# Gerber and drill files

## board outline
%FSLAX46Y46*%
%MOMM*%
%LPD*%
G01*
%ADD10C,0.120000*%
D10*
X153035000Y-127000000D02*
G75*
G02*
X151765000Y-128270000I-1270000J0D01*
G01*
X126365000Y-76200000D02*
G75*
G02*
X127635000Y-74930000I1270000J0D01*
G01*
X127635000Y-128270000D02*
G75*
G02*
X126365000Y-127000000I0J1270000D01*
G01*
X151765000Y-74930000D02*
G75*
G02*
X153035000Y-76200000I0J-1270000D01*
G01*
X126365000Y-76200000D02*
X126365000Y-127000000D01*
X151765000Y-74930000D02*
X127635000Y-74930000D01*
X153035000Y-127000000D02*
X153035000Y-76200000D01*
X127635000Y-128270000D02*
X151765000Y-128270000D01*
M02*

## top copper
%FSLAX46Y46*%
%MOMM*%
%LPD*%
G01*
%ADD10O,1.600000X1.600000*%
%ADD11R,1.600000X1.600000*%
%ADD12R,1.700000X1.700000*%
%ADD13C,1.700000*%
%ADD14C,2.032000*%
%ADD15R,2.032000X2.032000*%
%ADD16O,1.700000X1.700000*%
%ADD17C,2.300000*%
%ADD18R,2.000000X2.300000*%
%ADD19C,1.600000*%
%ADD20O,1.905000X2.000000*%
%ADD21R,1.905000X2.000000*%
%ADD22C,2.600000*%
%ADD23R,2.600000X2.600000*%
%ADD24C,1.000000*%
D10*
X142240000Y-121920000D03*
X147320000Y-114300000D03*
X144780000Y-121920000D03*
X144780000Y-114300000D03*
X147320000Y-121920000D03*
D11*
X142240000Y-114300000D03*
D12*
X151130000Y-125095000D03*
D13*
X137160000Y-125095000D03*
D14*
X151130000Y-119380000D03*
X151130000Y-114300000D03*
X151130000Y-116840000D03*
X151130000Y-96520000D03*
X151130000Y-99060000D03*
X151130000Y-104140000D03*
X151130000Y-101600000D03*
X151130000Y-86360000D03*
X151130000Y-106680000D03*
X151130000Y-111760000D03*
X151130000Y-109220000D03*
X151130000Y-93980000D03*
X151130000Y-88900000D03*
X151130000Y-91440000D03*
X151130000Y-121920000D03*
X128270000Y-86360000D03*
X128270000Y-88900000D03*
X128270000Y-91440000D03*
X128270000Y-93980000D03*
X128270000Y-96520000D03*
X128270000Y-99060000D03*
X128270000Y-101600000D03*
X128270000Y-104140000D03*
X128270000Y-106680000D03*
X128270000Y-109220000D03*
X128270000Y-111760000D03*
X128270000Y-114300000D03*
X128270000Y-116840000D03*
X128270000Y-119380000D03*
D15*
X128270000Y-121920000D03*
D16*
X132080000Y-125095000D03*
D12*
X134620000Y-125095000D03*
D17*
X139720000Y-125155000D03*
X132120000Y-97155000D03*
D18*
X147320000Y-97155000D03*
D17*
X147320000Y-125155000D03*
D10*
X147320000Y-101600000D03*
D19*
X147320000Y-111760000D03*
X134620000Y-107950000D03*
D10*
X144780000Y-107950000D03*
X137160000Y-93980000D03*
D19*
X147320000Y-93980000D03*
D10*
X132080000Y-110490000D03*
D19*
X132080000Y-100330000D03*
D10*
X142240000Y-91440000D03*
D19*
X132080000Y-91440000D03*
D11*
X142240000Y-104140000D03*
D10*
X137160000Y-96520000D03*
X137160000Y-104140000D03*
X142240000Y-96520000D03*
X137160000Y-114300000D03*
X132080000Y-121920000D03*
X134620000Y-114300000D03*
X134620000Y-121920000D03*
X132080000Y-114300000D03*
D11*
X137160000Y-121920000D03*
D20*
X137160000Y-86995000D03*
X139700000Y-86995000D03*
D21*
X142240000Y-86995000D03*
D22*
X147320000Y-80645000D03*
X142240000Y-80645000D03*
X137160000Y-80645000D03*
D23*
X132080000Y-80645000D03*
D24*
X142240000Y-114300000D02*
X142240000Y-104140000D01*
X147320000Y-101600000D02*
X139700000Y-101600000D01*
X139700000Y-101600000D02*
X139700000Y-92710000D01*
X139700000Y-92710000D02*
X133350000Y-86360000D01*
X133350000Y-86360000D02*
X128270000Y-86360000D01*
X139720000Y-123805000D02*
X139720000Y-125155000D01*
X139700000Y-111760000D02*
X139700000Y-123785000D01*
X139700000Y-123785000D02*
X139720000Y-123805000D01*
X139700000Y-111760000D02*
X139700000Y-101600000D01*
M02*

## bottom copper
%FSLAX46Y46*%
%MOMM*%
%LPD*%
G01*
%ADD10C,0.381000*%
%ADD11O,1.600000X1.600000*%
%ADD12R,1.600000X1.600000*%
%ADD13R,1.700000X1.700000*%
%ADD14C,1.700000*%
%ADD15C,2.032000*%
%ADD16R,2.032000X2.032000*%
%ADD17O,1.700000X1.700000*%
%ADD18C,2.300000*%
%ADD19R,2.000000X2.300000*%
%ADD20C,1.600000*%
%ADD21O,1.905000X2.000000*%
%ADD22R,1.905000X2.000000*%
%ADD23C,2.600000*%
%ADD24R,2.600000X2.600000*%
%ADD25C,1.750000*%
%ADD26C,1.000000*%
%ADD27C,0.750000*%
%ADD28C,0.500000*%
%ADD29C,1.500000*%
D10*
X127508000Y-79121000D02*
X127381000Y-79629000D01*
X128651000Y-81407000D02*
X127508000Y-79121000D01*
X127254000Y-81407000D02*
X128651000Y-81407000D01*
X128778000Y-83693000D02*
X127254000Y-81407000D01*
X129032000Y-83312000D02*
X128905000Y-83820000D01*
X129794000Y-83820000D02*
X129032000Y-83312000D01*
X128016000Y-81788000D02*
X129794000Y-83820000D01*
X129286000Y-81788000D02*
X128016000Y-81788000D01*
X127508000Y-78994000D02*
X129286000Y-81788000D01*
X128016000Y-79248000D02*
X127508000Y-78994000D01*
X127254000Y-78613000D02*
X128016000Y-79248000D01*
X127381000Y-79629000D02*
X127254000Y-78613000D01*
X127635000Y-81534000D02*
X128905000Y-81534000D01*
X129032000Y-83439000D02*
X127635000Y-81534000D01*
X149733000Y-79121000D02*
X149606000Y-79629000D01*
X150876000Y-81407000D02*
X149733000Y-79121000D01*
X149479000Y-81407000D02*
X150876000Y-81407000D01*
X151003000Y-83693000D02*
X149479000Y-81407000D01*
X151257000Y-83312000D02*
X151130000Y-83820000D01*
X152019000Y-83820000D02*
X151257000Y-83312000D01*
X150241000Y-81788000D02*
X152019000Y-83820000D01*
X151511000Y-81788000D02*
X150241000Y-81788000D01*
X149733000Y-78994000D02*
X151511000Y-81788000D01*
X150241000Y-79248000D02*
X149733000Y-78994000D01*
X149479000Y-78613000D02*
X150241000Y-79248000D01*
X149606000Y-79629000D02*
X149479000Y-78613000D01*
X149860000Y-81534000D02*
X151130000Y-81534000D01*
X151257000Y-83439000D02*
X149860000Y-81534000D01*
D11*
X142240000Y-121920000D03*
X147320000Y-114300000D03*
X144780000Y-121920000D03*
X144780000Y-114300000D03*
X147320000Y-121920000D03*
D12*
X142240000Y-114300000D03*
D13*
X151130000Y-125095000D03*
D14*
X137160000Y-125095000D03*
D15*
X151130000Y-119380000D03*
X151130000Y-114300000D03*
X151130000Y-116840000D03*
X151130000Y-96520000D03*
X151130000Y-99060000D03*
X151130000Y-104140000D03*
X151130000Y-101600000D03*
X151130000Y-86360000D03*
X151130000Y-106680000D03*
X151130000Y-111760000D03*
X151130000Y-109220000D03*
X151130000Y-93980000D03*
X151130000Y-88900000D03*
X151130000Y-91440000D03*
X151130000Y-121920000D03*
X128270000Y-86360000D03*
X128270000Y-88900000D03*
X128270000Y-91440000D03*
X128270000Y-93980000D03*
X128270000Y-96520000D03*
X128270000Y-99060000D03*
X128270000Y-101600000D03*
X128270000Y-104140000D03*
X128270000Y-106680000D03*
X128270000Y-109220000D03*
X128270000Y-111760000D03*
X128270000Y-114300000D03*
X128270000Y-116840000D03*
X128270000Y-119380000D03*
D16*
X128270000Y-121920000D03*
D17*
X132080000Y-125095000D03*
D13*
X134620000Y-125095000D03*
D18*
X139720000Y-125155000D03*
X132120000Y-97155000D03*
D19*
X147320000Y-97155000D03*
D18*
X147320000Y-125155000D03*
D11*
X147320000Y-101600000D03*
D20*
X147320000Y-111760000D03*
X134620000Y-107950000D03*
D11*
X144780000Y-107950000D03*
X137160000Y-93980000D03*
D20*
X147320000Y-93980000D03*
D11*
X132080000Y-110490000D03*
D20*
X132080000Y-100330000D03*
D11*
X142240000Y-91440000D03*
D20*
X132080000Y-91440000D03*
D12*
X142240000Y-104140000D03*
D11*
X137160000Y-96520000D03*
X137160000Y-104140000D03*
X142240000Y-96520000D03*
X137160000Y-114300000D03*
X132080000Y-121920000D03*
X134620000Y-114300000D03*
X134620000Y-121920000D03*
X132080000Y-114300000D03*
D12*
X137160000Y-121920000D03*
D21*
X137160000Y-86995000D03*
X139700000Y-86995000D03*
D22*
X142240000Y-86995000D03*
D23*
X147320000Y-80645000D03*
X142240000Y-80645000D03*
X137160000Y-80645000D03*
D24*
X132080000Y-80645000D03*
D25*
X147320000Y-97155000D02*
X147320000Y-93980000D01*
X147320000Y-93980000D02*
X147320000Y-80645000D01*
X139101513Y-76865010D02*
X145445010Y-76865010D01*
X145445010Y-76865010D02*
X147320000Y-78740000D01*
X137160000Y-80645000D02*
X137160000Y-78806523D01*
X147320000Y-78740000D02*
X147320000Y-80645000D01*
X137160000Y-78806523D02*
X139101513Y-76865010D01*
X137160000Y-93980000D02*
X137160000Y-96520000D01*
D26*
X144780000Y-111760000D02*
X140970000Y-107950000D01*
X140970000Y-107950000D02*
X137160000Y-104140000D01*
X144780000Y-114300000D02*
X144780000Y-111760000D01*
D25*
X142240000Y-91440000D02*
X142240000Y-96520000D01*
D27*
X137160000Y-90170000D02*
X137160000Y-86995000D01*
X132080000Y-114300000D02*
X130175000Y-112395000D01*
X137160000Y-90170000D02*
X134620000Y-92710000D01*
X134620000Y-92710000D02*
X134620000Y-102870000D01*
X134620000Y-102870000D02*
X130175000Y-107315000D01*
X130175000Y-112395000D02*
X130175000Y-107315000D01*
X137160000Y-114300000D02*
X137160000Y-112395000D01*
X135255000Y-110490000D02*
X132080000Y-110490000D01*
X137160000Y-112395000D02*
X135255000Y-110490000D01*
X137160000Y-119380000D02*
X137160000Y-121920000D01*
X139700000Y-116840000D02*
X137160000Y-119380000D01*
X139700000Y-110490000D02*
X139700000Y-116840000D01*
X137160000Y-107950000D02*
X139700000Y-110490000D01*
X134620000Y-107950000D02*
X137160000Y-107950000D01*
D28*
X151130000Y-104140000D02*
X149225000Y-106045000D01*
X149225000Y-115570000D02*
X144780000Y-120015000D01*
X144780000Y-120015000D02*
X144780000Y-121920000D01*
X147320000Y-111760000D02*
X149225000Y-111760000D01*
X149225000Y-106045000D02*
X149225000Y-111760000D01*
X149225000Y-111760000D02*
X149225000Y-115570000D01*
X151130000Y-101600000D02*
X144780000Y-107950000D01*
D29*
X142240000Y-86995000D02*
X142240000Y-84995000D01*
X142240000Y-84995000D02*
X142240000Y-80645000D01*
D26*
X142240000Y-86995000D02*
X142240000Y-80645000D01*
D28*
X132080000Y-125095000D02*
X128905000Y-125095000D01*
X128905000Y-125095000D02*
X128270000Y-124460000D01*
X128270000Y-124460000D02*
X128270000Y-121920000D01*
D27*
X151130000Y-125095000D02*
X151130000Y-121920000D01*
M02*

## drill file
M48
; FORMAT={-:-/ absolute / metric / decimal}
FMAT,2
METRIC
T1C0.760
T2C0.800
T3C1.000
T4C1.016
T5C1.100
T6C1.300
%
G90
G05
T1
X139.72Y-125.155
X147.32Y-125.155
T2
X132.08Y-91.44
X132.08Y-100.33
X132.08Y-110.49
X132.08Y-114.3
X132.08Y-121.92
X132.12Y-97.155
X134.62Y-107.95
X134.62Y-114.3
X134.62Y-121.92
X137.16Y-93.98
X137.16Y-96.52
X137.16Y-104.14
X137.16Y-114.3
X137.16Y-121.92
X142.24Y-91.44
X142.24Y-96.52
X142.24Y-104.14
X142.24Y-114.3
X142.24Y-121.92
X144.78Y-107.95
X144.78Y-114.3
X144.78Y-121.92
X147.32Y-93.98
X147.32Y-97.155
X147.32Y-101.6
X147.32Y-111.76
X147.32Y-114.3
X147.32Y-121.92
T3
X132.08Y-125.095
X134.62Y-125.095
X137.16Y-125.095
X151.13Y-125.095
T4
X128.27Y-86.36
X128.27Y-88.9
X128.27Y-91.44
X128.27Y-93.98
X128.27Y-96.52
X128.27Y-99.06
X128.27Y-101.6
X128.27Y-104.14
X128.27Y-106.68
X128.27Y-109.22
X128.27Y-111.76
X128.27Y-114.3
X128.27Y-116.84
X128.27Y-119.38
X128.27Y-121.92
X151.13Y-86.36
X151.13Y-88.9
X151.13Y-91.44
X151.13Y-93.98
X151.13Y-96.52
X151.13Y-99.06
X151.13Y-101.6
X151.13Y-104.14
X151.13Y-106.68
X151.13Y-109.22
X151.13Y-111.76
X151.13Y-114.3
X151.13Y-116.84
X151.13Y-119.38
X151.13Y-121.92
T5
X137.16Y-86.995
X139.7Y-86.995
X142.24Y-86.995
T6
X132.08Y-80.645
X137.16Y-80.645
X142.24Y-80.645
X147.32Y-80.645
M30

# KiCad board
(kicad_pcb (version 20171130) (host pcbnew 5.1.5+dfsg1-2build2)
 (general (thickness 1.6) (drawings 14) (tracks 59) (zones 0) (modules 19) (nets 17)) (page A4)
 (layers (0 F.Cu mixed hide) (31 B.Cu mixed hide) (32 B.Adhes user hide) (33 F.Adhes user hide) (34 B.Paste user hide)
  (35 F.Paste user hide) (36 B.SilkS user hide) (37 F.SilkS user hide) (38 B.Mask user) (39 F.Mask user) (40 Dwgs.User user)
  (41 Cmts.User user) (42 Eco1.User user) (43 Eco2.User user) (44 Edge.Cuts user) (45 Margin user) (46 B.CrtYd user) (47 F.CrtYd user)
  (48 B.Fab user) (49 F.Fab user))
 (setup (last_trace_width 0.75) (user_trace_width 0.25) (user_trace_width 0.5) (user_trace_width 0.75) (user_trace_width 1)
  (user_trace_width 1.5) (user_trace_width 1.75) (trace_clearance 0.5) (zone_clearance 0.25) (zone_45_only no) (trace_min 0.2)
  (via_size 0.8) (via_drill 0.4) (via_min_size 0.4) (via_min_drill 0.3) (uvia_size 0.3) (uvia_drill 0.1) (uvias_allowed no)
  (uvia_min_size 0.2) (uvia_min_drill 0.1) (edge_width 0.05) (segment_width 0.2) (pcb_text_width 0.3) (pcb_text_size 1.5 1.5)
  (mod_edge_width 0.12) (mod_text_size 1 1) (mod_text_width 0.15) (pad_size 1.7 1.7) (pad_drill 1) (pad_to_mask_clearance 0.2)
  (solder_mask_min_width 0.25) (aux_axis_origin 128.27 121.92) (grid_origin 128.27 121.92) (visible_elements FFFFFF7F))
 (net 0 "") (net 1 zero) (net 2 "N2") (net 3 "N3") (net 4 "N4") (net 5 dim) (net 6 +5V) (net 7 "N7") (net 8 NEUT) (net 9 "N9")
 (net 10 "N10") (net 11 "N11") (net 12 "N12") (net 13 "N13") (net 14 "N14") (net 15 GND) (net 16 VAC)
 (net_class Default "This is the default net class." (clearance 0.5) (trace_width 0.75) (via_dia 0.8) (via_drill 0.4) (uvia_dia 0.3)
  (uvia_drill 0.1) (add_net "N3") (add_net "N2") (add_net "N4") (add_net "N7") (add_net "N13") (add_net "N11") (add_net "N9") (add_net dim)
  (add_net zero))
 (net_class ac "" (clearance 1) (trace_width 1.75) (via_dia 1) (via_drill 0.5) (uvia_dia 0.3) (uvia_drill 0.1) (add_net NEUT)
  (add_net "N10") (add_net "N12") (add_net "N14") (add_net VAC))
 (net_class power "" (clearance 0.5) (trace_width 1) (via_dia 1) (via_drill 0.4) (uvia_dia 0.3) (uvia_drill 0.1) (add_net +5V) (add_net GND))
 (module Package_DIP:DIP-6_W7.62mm (layer B.Cu) (at 142.24 114.3 270)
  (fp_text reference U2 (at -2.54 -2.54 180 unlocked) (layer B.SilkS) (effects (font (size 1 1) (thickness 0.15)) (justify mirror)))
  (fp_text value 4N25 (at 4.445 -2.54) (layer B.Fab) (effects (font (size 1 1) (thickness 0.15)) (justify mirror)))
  (pad 6 thru_hole oval (at 7.62 0 270) (size 1.6 1.6) (drill 0.8) (layers *.Cu *.Mask))
  (pad 3 thru_hole oval (at 0 -5.08 270) (size 1.6 1.6) (drill 0.8) (layers *.Cu *.Mask))
  (pad 5 thru_hole oval (at 7.62 -2.54 270) (size 1.6 1.6) (drill 0.8) (layers *.Cu *.Mask) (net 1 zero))
  (pad 2 thru_hole oval (at 0 -2.54 270) (size 1.6 1.6) (drill 0.8) (layers *.Cu *.Mask) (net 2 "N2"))
  (pad 4 thru_hole oval (at 7.62 -5.08 270) (size 1.6 1.6) (drill 0.8) (layers *.Cu *.Mask))
  (pad 1 thru_hole rect (at 0 0 270) (size 1.6 1.6) (drill 0.8) (layers *.Cu *.Mask) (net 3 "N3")))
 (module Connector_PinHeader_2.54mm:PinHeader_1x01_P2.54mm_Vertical (layer B.Cu) (at 151.13 125.095)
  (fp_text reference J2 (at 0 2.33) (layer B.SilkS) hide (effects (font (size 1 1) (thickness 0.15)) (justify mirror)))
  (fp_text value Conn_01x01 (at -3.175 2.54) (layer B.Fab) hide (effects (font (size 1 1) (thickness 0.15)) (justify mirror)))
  (pad 1 thru_hole rect (at 0 0) (size 1.7 1.7) (drill 1) (layers *.Cu *.Mask) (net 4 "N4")))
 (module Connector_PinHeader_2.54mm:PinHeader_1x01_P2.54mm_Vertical (layer B.Cu) (at 137.16 125.095)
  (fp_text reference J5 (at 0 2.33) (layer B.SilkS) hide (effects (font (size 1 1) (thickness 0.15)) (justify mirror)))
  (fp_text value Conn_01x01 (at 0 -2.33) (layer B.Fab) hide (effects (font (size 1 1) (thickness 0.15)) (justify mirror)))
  (pad 1 thru_hole circle (at 0 0) (size 1.7 1.7) (drill 1) (layers *.Cu *.Mask)))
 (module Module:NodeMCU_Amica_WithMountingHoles (layer B.Cu) (at 128.27 121.92)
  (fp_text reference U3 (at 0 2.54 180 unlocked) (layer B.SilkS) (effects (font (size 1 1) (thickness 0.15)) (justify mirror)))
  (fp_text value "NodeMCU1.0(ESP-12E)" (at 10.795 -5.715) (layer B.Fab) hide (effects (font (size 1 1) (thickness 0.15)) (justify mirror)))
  (pad 29 thru_hole circle (at 22.86 -2.54) (size 2.032 2.032) (drill 1.016) (layers *.Cu *.Mask))
  (pad 27 thru_hole circle (at 22.86 -7.62) (size 2.032 2.032) (drill 1.016) (layers *.Cu *.Mask))
  (pad 28 thru_hole circle (at 22.86 -5.08) (size 2.032 2.032) (drill 1.016) (layers *.Cu *.Mask))
  (pad 20 thru_hole circle (at 22.86 -25.4) (size 2.032 2.032) (drill 1.016) (layers *.Cu *.Mask))
  (pad 21 thru_hole circle (at 22.86 -22.86) (size 2.032 2.032) (drill 1.016) (layers *.Cu *.Mask))
  (pad 23 thru_hole circle (at 22.86 -17.78) (size 2.032 2.032) (drill 1.016) (layers *.Cu *.Mask) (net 1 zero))
  (pad 22 thru_hole circle (at 22.86 -20.32) (size 2.032 2.032) (drill 1.016) (layers *.Cu *.Mask) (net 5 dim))
  (pad 16 thru_hole circle (at 22.86 -35.56) (size 2.032 2.032) (drill 1.016) (layers *.Cu *.Mask))
  (pad 24 thru_hole circle (at 22.86 -15.24) (size 2.032 2.032) (drill 1.016) (layers *.Cu *.Mask))
  (pad 26 thru_hole circle (at 22.86 -10.16) (size 2.032 2.032) (drill 1.016) (layers *.Cu *.Mask))
  (pad 25 thru_hole circle (at 22.86 -12.7) (size 2.032 2.032) (drill 1.016) (layers *.Cu *.Mask))
  (pad 19 thru_hole circle (at 22.86 -27.94) (size 2.032 2.032) (drill 1.016) (layers *.Cu *.Mask))
  (pad 17 thru_hole circle (at 22.86 -33.02) (size 2.032 2.032) (drill 1.016) (layers *.Cu *.Mask))
  (pad 18 thru_hole circle (at 22.86 -30.48) (size 2.032 2.032) (drill 1.016) (layers *.Cu *.Mask))
  (pad 30 thru_hole circle (at 22.86 0) (size 2.032 2.032) (drill 1.016) (layers *.Cu *.Mask) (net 4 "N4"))
  (pad 15 thru_hole circle (at 0 -35.56) (size 2.032 2.032) (drill 1.016) (layers *.Cu *.Mask) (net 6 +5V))
  (pad 14 thru_hole circle (at 0 -33.02) (size 2.032 2.032) (drill 1.016) (layers *.Cu *.Mask))
  (pad 13 thru_hole circle (at 0 -30.48) (size 2.032 2.032) (drill 1.016) (layers *.Cu *.Mask))
  (pad 12 thru_hole circle (at 0 -27.94) (size 2.032 2.032) (drill 1.016) (layers *.Cu *.Mask))
  (pad 11 thru_hole circle (at 0 -25.4) (size 2.032 2.032) (drill 1.016) (layers *.Cu *.Mask))
  (pad 10 thru_hole circle (at 0 -22.86) (size 2.032 2.032) (drill 1.016) (layers *.Cu *.Mask))
  (pad 9 thru_hole circle (at 0 -20.32) (size 2.032 2.032) (drill 1.016) (layers *.Cu *.Mask))
  (pad 8 thru_hole circle (at 0 -17.78) (size 2.032 2.032) (drill 1.016) (layers *.Cu *.Mask))
  (pad 7 thru_hole circle (at 0 -15.24) (size 2.032 2.032) (drill 1.016) (layers *.Cu *.Mask))
  (pad 6 thru_hole circle (at 0 -12.7) (size 2.032 2.032) (drill 1.016) (layers *.Cu *.Mask))
  (pad 5 thru_hole circle (at 0 -10.16) (size 2.032 2.032) (drill 1.016) (layers *.Cu *.Mask))
  (pad 4 thru_hole circle (at 0 -7.62) (size 2.032 2.032) (drill 1.016) (layers *.Cu *.Mask))
  (pad 3 thru_hole circle (at 0 -5.08) (size 2.032 2.032) (drill 1.016) (layers *.Cu *.Mask))
  (pad 2 thru_hole circle (at 0 -2.54) (size 2.032 2.032) (drill 1.016) (layers *.Cu *.Mask))
  (pad 1 thru_hole rect (at 0 0) (size 2.032 2.032) (drill 1.016) (layers *.Cu *.Mask) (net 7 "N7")))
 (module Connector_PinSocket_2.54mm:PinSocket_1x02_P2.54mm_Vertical (layer B.Cu) (at 134.62 125.095 90)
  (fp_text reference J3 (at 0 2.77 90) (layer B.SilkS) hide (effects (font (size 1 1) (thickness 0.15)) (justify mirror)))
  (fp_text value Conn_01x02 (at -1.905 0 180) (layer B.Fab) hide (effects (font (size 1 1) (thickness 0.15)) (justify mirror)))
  (pad 2 thru_hole oval (at 0 -2.54 90) (size 1.7 1.7) (drill 1) (layers *.Cu *.Mask) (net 7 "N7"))
  (pad 1 thru_hole rect (at 0 0 90) (size 1.7 1.7) (drill 1) (layers *.Cu *.Mask)))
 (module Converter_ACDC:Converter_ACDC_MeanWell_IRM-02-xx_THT (layer F.Cu) (at 147.32 97.155 270)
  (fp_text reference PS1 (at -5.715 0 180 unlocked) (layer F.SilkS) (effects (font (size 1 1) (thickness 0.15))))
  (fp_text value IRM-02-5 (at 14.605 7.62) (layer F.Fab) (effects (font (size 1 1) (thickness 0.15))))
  (pad 4 thru_hole circle (at 28 7.6 270) (size 2.3 2.3) (drill 0.76) (layers *.Cu *.Mask) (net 6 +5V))
  (pad 2 thru_hole circle (at 0 15.2 270) (size 2.3 2.3) (drill 0.8) (layers *.Cu *.Mask))
  (pad 1 thru_hole rect (at 0 0 270) (size 2.3 2) (drill 0.8) (layers *.Cu *.Mask) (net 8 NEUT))
  (pad 3 thru_hole circle (at 28 0 270) (size 2.3 2.3) (drill 0.76) (layers *.Cu *.Mask)))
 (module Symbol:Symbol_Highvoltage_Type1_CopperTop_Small (layer B.Cu) (at 127.635 80.645)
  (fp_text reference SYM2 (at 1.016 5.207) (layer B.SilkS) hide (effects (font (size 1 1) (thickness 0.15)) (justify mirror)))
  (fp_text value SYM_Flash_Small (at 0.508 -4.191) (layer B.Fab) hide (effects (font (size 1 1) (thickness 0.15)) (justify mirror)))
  (fp_line (start -0.127 -1.524) (end -0.254 -1.016) (layer B.Cu) (width 0.381))
  (fp_line (start 1.016 0.762) (end -0.127 -1.524) (layer B.Cu) (width 0.381))
  (fp_line (start -0.381 0.762) (end 1.016 0.762) (layer B.Cu) (width 0.381))
  (fp_line (start 1.143 3.048) (end -0.381 0.762) (layer B.Cu) (width 0.381))
  (fp_line (start 1.397 2.667) (end 1.27 3.175) (layer B.Cu) (width 0.381))
  (fp_line (start 2.159 3.175) (end 1.397 2.667) (layer B.Cu) (width 0.381))
  (fp_line (start 0.381 1.143) (end 2.159 3.175) (layer B.Cu) (width 0.381))
  (fp_line (start 1.651 1.143) (end 0.381 1.143) (layer B.Cu) (width 0.381))
  (fp_line (start -0.127 -1.651) (end 1.651 1.143) (layer B.Cu) (width 0.381))
  (fp_line (start 0.381 -1.397) (end -0.127 -1.651) (layer B.Cu) (width 0.381))
  (fp_line (start -0.381 -2.032) (end 0.381 -1.397) (layer B.Cu) (width 0.381))
  (fp_line (start -0.254 -1.016) (end -0.381 -2.032) (layer B.Cu) (width 0.381))
  (fp_line (start 0 0.889) (end 1.27 0.889) (layer B.Cu) (width 0.381))
  (fp_line (start 1.397 2.794) (end 0 0.889) (layer B.Cu) (width 0.381)))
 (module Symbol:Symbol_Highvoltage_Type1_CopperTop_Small (layer B.Cu) (at 149.86 80.645)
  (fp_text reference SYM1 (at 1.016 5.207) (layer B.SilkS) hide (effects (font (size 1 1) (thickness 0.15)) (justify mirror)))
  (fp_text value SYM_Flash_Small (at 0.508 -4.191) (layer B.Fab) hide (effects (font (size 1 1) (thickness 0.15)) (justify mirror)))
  (fp_line (start -0.127 -1.524) (end -0.254 -1.016) (layer B.Cu) (width 0.381))
  (fp_line (start 1.016 0.762) (end -0.127 -1.524) (layer B.Cu) (width 0.381))
  (fp_line (start -0.381 0.762) (end 1.016 0.762) (layer B.Cu) (width 0.381))
  (fp_line (start 1.143 3.048) (end -0.381 0.762) (layer B.Cu) (width 0.381))
  (fp_line (start 1.397 2.667) (end 1.27 3.175) (layer B.Cu) (width 0.381))
  (fp_line (start 2.159 3.175) (end 1.397 2.667) (layer B.Cu) (width 0.381))
  (fp_line (start 0.381 1.143) (end 2.159 3.175) (layer B.Cu) (width 0.381))
  (fp_line (start 1.651 1.143) (end 0.381 1.143) (layer B.Cu) (width 0.381))
  (fp_line (start -0.127 -1.651) (end 1.651 1.143) (layer B.Cu) (width 0.381))
  (fp_line (start 0.381 -1.397) (end -0.127 -1.651) (layer B.Cu) (width 0.381))
  (fp_line (start -0.381 -2.032) (end 0.381 -1.397) (layer B.Cu) (width 0.381))
  (fp_line (start -0.254 -1.016) (end -0.381 -2.032) (layer B.Cu) (width 0.381))
  (fp_line (start 0 0.889) (end 1.27 0.889) (layer B.Cu) (width 0.381))
  (fp_line (start 1.397 2.794) (end 0 0.889) (layer B.Cu) (width 0.381)))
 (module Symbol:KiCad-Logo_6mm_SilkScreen (layer F.Cu) (at 143.51 105.41 90)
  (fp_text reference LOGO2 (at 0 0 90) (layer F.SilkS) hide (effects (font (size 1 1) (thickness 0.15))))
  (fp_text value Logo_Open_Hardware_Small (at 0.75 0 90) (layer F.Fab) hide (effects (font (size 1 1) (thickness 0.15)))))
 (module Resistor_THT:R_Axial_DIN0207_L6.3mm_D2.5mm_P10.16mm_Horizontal (layer B.Cu) (at 147.32 111.76 90)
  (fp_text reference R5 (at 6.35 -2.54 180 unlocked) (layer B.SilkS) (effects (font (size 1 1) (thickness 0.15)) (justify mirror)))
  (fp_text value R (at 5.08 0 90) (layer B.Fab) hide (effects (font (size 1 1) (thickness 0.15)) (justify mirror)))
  (pad 2 thru_hole oval (at 10.16 0 90) (size 1.6 1.6) (drill 0.8) (layers *.Cu *.Mask) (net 6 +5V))
  (pad 1 thru_hole circle (at 0 0 90) (size 1.6 1.6) (drill 0.8) (layers *.Cu *.Mask) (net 1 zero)))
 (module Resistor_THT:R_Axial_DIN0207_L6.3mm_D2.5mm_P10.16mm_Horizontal (layer B.Cu) (at 134.62 107.95)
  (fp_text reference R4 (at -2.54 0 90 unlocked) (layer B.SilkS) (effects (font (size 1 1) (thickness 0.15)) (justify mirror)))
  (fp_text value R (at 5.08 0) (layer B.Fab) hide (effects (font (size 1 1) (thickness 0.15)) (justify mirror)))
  (pad 1 thru_hole circle (at 0 0) (size 1.6 1.6) (drill 0.8) (layers *.Cu *.Mask) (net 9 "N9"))
  (pad 2 thru_hole oval (at 10.16 0) (size 1.6 1.6) (drill 0.8) (layers *.Cu *.Mask) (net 5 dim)))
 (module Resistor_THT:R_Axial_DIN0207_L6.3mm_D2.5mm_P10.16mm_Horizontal (layer B.Cu) (at 147.32 93.98 180)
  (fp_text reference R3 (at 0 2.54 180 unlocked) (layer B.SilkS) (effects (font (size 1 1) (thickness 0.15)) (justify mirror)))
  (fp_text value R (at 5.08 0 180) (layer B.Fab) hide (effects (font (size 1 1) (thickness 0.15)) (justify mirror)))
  (pad 2 thru_hole oval (at 10.16 0 180) (size 1.6 1.6) (drill 0.8) (layers *.Cu *.Mask) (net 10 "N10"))
  (pad 1 thru_hole circle (at 0 0 180) (size 1.6 1.6) (drill 0.8) (layers *.Cu *.Mask) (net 8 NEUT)))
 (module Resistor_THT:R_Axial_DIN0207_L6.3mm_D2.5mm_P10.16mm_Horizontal (layer B.Cu) (at 132.08 100.33 270)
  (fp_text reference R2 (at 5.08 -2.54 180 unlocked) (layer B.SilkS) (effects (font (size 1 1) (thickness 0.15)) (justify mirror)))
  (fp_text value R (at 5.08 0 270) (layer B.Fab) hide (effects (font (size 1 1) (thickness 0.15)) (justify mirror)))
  (pad 2 thru_hole oval (at 10.16 0 270) (size 1.6 1.6) (drill 0.8) (layers *.Cu *.Mask) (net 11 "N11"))
  (pad 1 thru_hole circle (at 0 0 270) (size 1.6 1.6) (drill 0.8) (layers *.Cu *.Mask)))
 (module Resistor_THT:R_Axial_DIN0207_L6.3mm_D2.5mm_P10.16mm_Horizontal (layer B.Cu) (at 132.08 91.44)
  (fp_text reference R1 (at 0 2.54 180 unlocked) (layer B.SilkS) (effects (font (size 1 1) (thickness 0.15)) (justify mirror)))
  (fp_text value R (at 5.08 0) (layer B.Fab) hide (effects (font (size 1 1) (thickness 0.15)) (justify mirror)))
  (pad 2 thru_hole oval (at 10.16 0) (size 1.6 1.6) (drill 0.8) (layers *.Cu *.Mask) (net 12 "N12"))
  (pad 1 thru_hole circle (at 0 0) (size 1.6 1.6) (drill 0.8) (layers *.Cu *.Mask)))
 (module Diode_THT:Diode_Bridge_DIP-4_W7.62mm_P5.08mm (layer B.Cu) (at 142.24 104.14 90)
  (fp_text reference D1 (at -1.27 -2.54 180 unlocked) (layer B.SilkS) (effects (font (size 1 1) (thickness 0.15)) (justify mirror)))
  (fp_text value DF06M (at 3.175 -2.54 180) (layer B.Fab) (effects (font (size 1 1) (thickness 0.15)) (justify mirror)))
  (pad 1 thru_hole rect (at 0 0 90) (size 1.6 1.6) (drill 0.8) (layers *.Cu *.Mask) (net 3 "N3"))
  (pad 3 thru_hole oval (at 7.62 -5.08 90) (size 1.6 1.6) (drill 0.8) (layers *.Cu *.Mask) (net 10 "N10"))
  (pad 2 thru_hole oval (at 0 -5.08 90) (size 1.6 1.6) (drill 0.8) (layers *.Cu *.Mask) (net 2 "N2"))
  (pad 4 thru_hole oval (at 7.62 0 90) (size 1.6 1.6) (drill 0.8) (layers *.Cu *.Mask) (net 12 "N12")))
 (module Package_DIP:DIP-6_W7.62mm (layer B.Cu) (at 137.16 121.92 90)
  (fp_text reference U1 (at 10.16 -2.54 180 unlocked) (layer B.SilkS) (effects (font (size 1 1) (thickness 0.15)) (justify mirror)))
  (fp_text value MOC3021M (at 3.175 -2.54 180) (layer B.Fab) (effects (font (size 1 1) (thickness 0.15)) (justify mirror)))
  (pad 6 thru_hole oval (at 7.62 0 90) (size 1.6 1.6) (drill 0.8) (layers *.Cu *.Mask) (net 11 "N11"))
  (pad 3 thru_hole oval (at 0 -5.08 90) (size 1.6 1.6) (drill 0.8) (layers *.Cu *.Mask))
  (pad 5 thru_hole oval (at 7.62 -2.54 90) (size 1.6 1.6) (drill 0.8) (layers *.Cu *.Mask))
  (pad 2 thru_hole oval (at 0 -2.54 90) (size 1.6 1.6) (drill 0.8) (layers *.Cu *.Mask))
  (pad 4 thru_hole oval (at 7.62 -5.08 90) (size 1.6 1.6) (drill 0.8) (layers *.Cu *.Mask) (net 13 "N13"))
  (pad 1 thru_hole rect (at 0 0 90) (size 1.6 1.6) (drill 0.8) (layers *.Cu *.Mask) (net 9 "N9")))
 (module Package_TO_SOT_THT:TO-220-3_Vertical (layer F.Cu) (at 142.24 86.995 180)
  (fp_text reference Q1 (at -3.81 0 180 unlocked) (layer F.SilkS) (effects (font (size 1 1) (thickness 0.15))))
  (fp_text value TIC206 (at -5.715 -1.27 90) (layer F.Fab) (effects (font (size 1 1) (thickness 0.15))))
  (pad 3 thru_hole oval (at 5.08 0 180) (size 1.905 2) (drill 1.1) (layers *.Cu *.Mask) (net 13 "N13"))
  (pad 2 thru_hole oval (at 2.54 0 180) (size 1.905 2) (drill 1.1) (layers *.Cu *.Mask))
  (pad 1 thru_hole rect (at 0 0 180) (size 1.905 2) (drill 1.1) (layers *.Cu *.Mask) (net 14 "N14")))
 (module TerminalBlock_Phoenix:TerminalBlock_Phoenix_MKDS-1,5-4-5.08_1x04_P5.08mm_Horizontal (layer F.Cu) (at 132.08 80.645)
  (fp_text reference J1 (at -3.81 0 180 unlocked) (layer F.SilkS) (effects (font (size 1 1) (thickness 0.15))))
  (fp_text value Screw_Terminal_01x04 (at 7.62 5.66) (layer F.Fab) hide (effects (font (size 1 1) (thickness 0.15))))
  (pad 4 thru_hole circle (at 15.24 0) (size 2.6 2.6) (drill 1.3) (layers *.Cu *.Mask) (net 8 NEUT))
  (pad 3 thru_hole circle (at 10.16 0) (size 2.6 2.6) (drill 1.3) (layers *.Cu *.Mask) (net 14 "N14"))
  (pad 2 thru_hole circle (at 5.08 0) (size 2.6 2.6) (drill 1.3) (layers *.Cu *.Mask) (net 8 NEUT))
  (pad 1 thru_hole rect (at 0 0) (size 2.6 2.6) (drill 1.3) (layers *.Cu *.Mask)))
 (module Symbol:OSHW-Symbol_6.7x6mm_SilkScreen (layer F.Cu) (at 143.51 118.11 90)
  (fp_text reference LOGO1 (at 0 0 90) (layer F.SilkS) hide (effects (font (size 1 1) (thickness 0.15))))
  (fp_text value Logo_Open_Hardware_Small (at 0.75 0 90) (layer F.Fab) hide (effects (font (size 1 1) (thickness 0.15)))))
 (gr_arc (start 151.765 127) (end 151.765 128.27) (angle -90) (layer Edge.Cuts) (width 0.12))
 (gr_arc (start 127.635 76.2) (end 127.635 74.93) (angle -90) (layer Edge.Cuts) (width 0.12))
 (gr_arc (start 127.635 127) (end 126.365 127) (angle -90) (layer Edge.Cuts) (width 0.12))
 (gr_arc (start 151.765 76.2) (end 153.035 76.2) (angle -90) (layer Edge.Cuts) (width 0.12))
 (gr_line (start 126.365 76.2) (end 126.365 127) (layer Edge.Cuts) (width 0.12))
 (gr_line (start 151.765 74.93) (end 127.635 74.93) (layer Edge.Cuts) (width 0.12))
 (gr_line (start 153.035 127) (end 153.035 76.2) (layer Edge.Cuts) (width 0.12))
 (gr_line (start 127.635 128.27) (end 151.765 128.27) (layer Edge.Cuts) (width 0.12))
 (segment (start 147.32 97.155) (end 147.32 93.98) (width 1.75) (layer B.Cu) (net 8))
 (segment (start 147.32 93.98) (end 147.32 80.645) (width 1.75) (layer B.Cu) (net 8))
 (segment (start 139.101513 76.86501) (end 145.44501 76.86501) (width 1.75) (layer B.Cu) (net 8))
 (segment (start 145.44501 76.86501) (end 147.32 78.74) (width 1.75) (layer B.Cu) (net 8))
 (segment (start 137.16 80.645) (end 137.16 78.806523) (width 1.75) (layer B.Cu) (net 8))
 (segment (start 147.32 78.74) (end 147.32 80.645) (width 1.75) (layer B.Cu) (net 8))
 (segment (start 137.16 78.806523) (end 139.101513 76.86501) (width 1.75) (layer B.Cu) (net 8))
 (segment (start 142.24 114.3) (end 142.24 104.14) (width 1) (layer F.Cu) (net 3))
 (segment (start 137.16 93.98) (end 137.16 96.52) (width 1.75) (layer B.Cu) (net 10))
 (segment (start 144.78 111.76) (end 140.97 107.95) (width 1) (layer B.Cu) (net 2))
 (segment (start 140.97 107.95) (end 137.16 104.14) (width 1) (layer B.Cu) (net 2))
 (segment (start 144.78 114.3) (end 144.78 111.76) (width 1) (layer B.Cu) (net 2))
 (segment (start 142.24 91.44) (end 142.24 96.52) (width 1.75) (layer B.Cu) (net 12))
 (segment (start 137.16 90.17) (end 137.16 86.995) (width 0.75) (layer B.Cu) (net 13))
 (segment (start 132.08 114.3) (end 130.175 112.395) (width 0.75) (layer B.Cu) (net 13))
 (segment (start 137.16 90.17) (end 134.62 92.71) (width 0.75) (layer B.Cu) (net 13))
 (segment (start 134.62 92.71) (end 134.62 102.87) (width 0.75) (layer B.Cu) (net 13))
 (segment (start 134.62 102.87) (end 130.175 107.315) (width 0.75) (layer B.Cu) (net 13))
 (segment (start 130.175 112.395) (end 130.175 107.315) (width 0.75) (layer B.Cu) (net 13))
 (segment (start 137.16 114.3) (end 137.16 112.395) (width 0.75) (layer B.Cu) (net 11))
 (segment (start 135.255 110.49) (end 132.08 110.49) (width 0.75) (layer B.Cu) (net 11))
 (segment (start 137.16 112.395) (end 135.255 110.49) (width 0.75) (layer B.Cu) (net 11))
 (segment (start 137.16 119.38) (end 137.16 121.92) (width 0.75) (layer B.Cu) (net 9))
 (segment (start 139.7 116.84) (end 137.16 119.38) (width 0.75) (layer B.Cu) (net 9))
 (segment (start 139.7 110.49) (end 139.7 116.84) (width 0.75) (layer B.Cu) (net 9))
 (segment (start 137.16 107.95) (end 139.7 110.49) (width 0.75) (layer B.Cu) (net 9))
 (segment (start 134.62 107.95) (end 137.16 107.95) (width 0.75) (layer B.Cu) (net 9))
 (segment (start 151.13 104.14) (end 149.225 106.045) (width 0.5) (layer B.Cu) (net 1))
 (segment (start 149.225 115.57) (end 144.78 120.015) (width 0.5) (layer B.Cu) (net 1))
 (segment (start 144.78 120.015) (end 144.78 121.92) (width 0.5) (layer B.Cu) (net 1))
 (segment (start 147.32 111.76) (end 149.225 111.76) (width 0.5) (layer B.Cu) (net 1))
 (segment (start 149.225 106.045) (end 149.225 111.76) (width 0.5) (layer B.Cu) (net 1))
 (segment (start 149.225 111.76) (end 149.225 115.57) (width 0.5) (layer B.Cu) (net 1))
 (segment (start 151.13 101.6) (end 144.78 107.95) (width 0.5) (layer B.Cu) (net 5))
 (segment (start 147.32 101.6) (end 139.7 101.6) (width 1) (layer F.Cu) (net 6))
 (segment (start 139.7 101.6) (end 139.7 92.71) (width 1) (layer F.Cu) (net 6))
 (segment (start 139.7 92.71) (end 133.35 86.36) (width 1) (layer F.Cu) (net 6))
 (segment (start 133.35 86.36) (end 128.27 86.36) (width 1) (layer F.Cu) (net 6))
 (segment (start 139.72 123.805) (end 139.72 125.155) (width 1) (layer F.Cu) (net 6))
 (segment (start 139.7 111.76) (end 139.7 123.785) (width 1) (layer F.Cu) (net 6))
 (segment (start 139.7 123.785) (end 139.72 123.805) (width 1) (layer F.Cu) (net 6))
 (segment (start 139.7 111.76) (end 139.7 101.6) (width 1) (layer F.Cu) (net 6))
 (segment (start 142.24 86.995) (end 142.24 84.995) (width 1.5) (layer B.Cu) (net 14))
 (segment (start 142.24 84.995) (end 142.24 80.645) (width 1.5) (layer B.Cu) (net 14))
 (segment (start 142.24 86.995) (end 142.24 80.645) (width 1) (layer B.Cu) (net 14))
 (segment (start 132.08 125.095) (end 128.905 125.095) (width 0.5) (layer B.Cu) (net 7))
 (segment (start 128.905 125.095) (end 128.27 124.46) (width 0.5) (layer B.Cu) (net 7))
 (segment (start 128.27 124.46) (end 128.27 121.92) (width 0.5) (layer B.Cu) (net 7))
 (segment (start 151.13 125.095) (end 151.13 121.92) (width 0.75) (layer B.Cu) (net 4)))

